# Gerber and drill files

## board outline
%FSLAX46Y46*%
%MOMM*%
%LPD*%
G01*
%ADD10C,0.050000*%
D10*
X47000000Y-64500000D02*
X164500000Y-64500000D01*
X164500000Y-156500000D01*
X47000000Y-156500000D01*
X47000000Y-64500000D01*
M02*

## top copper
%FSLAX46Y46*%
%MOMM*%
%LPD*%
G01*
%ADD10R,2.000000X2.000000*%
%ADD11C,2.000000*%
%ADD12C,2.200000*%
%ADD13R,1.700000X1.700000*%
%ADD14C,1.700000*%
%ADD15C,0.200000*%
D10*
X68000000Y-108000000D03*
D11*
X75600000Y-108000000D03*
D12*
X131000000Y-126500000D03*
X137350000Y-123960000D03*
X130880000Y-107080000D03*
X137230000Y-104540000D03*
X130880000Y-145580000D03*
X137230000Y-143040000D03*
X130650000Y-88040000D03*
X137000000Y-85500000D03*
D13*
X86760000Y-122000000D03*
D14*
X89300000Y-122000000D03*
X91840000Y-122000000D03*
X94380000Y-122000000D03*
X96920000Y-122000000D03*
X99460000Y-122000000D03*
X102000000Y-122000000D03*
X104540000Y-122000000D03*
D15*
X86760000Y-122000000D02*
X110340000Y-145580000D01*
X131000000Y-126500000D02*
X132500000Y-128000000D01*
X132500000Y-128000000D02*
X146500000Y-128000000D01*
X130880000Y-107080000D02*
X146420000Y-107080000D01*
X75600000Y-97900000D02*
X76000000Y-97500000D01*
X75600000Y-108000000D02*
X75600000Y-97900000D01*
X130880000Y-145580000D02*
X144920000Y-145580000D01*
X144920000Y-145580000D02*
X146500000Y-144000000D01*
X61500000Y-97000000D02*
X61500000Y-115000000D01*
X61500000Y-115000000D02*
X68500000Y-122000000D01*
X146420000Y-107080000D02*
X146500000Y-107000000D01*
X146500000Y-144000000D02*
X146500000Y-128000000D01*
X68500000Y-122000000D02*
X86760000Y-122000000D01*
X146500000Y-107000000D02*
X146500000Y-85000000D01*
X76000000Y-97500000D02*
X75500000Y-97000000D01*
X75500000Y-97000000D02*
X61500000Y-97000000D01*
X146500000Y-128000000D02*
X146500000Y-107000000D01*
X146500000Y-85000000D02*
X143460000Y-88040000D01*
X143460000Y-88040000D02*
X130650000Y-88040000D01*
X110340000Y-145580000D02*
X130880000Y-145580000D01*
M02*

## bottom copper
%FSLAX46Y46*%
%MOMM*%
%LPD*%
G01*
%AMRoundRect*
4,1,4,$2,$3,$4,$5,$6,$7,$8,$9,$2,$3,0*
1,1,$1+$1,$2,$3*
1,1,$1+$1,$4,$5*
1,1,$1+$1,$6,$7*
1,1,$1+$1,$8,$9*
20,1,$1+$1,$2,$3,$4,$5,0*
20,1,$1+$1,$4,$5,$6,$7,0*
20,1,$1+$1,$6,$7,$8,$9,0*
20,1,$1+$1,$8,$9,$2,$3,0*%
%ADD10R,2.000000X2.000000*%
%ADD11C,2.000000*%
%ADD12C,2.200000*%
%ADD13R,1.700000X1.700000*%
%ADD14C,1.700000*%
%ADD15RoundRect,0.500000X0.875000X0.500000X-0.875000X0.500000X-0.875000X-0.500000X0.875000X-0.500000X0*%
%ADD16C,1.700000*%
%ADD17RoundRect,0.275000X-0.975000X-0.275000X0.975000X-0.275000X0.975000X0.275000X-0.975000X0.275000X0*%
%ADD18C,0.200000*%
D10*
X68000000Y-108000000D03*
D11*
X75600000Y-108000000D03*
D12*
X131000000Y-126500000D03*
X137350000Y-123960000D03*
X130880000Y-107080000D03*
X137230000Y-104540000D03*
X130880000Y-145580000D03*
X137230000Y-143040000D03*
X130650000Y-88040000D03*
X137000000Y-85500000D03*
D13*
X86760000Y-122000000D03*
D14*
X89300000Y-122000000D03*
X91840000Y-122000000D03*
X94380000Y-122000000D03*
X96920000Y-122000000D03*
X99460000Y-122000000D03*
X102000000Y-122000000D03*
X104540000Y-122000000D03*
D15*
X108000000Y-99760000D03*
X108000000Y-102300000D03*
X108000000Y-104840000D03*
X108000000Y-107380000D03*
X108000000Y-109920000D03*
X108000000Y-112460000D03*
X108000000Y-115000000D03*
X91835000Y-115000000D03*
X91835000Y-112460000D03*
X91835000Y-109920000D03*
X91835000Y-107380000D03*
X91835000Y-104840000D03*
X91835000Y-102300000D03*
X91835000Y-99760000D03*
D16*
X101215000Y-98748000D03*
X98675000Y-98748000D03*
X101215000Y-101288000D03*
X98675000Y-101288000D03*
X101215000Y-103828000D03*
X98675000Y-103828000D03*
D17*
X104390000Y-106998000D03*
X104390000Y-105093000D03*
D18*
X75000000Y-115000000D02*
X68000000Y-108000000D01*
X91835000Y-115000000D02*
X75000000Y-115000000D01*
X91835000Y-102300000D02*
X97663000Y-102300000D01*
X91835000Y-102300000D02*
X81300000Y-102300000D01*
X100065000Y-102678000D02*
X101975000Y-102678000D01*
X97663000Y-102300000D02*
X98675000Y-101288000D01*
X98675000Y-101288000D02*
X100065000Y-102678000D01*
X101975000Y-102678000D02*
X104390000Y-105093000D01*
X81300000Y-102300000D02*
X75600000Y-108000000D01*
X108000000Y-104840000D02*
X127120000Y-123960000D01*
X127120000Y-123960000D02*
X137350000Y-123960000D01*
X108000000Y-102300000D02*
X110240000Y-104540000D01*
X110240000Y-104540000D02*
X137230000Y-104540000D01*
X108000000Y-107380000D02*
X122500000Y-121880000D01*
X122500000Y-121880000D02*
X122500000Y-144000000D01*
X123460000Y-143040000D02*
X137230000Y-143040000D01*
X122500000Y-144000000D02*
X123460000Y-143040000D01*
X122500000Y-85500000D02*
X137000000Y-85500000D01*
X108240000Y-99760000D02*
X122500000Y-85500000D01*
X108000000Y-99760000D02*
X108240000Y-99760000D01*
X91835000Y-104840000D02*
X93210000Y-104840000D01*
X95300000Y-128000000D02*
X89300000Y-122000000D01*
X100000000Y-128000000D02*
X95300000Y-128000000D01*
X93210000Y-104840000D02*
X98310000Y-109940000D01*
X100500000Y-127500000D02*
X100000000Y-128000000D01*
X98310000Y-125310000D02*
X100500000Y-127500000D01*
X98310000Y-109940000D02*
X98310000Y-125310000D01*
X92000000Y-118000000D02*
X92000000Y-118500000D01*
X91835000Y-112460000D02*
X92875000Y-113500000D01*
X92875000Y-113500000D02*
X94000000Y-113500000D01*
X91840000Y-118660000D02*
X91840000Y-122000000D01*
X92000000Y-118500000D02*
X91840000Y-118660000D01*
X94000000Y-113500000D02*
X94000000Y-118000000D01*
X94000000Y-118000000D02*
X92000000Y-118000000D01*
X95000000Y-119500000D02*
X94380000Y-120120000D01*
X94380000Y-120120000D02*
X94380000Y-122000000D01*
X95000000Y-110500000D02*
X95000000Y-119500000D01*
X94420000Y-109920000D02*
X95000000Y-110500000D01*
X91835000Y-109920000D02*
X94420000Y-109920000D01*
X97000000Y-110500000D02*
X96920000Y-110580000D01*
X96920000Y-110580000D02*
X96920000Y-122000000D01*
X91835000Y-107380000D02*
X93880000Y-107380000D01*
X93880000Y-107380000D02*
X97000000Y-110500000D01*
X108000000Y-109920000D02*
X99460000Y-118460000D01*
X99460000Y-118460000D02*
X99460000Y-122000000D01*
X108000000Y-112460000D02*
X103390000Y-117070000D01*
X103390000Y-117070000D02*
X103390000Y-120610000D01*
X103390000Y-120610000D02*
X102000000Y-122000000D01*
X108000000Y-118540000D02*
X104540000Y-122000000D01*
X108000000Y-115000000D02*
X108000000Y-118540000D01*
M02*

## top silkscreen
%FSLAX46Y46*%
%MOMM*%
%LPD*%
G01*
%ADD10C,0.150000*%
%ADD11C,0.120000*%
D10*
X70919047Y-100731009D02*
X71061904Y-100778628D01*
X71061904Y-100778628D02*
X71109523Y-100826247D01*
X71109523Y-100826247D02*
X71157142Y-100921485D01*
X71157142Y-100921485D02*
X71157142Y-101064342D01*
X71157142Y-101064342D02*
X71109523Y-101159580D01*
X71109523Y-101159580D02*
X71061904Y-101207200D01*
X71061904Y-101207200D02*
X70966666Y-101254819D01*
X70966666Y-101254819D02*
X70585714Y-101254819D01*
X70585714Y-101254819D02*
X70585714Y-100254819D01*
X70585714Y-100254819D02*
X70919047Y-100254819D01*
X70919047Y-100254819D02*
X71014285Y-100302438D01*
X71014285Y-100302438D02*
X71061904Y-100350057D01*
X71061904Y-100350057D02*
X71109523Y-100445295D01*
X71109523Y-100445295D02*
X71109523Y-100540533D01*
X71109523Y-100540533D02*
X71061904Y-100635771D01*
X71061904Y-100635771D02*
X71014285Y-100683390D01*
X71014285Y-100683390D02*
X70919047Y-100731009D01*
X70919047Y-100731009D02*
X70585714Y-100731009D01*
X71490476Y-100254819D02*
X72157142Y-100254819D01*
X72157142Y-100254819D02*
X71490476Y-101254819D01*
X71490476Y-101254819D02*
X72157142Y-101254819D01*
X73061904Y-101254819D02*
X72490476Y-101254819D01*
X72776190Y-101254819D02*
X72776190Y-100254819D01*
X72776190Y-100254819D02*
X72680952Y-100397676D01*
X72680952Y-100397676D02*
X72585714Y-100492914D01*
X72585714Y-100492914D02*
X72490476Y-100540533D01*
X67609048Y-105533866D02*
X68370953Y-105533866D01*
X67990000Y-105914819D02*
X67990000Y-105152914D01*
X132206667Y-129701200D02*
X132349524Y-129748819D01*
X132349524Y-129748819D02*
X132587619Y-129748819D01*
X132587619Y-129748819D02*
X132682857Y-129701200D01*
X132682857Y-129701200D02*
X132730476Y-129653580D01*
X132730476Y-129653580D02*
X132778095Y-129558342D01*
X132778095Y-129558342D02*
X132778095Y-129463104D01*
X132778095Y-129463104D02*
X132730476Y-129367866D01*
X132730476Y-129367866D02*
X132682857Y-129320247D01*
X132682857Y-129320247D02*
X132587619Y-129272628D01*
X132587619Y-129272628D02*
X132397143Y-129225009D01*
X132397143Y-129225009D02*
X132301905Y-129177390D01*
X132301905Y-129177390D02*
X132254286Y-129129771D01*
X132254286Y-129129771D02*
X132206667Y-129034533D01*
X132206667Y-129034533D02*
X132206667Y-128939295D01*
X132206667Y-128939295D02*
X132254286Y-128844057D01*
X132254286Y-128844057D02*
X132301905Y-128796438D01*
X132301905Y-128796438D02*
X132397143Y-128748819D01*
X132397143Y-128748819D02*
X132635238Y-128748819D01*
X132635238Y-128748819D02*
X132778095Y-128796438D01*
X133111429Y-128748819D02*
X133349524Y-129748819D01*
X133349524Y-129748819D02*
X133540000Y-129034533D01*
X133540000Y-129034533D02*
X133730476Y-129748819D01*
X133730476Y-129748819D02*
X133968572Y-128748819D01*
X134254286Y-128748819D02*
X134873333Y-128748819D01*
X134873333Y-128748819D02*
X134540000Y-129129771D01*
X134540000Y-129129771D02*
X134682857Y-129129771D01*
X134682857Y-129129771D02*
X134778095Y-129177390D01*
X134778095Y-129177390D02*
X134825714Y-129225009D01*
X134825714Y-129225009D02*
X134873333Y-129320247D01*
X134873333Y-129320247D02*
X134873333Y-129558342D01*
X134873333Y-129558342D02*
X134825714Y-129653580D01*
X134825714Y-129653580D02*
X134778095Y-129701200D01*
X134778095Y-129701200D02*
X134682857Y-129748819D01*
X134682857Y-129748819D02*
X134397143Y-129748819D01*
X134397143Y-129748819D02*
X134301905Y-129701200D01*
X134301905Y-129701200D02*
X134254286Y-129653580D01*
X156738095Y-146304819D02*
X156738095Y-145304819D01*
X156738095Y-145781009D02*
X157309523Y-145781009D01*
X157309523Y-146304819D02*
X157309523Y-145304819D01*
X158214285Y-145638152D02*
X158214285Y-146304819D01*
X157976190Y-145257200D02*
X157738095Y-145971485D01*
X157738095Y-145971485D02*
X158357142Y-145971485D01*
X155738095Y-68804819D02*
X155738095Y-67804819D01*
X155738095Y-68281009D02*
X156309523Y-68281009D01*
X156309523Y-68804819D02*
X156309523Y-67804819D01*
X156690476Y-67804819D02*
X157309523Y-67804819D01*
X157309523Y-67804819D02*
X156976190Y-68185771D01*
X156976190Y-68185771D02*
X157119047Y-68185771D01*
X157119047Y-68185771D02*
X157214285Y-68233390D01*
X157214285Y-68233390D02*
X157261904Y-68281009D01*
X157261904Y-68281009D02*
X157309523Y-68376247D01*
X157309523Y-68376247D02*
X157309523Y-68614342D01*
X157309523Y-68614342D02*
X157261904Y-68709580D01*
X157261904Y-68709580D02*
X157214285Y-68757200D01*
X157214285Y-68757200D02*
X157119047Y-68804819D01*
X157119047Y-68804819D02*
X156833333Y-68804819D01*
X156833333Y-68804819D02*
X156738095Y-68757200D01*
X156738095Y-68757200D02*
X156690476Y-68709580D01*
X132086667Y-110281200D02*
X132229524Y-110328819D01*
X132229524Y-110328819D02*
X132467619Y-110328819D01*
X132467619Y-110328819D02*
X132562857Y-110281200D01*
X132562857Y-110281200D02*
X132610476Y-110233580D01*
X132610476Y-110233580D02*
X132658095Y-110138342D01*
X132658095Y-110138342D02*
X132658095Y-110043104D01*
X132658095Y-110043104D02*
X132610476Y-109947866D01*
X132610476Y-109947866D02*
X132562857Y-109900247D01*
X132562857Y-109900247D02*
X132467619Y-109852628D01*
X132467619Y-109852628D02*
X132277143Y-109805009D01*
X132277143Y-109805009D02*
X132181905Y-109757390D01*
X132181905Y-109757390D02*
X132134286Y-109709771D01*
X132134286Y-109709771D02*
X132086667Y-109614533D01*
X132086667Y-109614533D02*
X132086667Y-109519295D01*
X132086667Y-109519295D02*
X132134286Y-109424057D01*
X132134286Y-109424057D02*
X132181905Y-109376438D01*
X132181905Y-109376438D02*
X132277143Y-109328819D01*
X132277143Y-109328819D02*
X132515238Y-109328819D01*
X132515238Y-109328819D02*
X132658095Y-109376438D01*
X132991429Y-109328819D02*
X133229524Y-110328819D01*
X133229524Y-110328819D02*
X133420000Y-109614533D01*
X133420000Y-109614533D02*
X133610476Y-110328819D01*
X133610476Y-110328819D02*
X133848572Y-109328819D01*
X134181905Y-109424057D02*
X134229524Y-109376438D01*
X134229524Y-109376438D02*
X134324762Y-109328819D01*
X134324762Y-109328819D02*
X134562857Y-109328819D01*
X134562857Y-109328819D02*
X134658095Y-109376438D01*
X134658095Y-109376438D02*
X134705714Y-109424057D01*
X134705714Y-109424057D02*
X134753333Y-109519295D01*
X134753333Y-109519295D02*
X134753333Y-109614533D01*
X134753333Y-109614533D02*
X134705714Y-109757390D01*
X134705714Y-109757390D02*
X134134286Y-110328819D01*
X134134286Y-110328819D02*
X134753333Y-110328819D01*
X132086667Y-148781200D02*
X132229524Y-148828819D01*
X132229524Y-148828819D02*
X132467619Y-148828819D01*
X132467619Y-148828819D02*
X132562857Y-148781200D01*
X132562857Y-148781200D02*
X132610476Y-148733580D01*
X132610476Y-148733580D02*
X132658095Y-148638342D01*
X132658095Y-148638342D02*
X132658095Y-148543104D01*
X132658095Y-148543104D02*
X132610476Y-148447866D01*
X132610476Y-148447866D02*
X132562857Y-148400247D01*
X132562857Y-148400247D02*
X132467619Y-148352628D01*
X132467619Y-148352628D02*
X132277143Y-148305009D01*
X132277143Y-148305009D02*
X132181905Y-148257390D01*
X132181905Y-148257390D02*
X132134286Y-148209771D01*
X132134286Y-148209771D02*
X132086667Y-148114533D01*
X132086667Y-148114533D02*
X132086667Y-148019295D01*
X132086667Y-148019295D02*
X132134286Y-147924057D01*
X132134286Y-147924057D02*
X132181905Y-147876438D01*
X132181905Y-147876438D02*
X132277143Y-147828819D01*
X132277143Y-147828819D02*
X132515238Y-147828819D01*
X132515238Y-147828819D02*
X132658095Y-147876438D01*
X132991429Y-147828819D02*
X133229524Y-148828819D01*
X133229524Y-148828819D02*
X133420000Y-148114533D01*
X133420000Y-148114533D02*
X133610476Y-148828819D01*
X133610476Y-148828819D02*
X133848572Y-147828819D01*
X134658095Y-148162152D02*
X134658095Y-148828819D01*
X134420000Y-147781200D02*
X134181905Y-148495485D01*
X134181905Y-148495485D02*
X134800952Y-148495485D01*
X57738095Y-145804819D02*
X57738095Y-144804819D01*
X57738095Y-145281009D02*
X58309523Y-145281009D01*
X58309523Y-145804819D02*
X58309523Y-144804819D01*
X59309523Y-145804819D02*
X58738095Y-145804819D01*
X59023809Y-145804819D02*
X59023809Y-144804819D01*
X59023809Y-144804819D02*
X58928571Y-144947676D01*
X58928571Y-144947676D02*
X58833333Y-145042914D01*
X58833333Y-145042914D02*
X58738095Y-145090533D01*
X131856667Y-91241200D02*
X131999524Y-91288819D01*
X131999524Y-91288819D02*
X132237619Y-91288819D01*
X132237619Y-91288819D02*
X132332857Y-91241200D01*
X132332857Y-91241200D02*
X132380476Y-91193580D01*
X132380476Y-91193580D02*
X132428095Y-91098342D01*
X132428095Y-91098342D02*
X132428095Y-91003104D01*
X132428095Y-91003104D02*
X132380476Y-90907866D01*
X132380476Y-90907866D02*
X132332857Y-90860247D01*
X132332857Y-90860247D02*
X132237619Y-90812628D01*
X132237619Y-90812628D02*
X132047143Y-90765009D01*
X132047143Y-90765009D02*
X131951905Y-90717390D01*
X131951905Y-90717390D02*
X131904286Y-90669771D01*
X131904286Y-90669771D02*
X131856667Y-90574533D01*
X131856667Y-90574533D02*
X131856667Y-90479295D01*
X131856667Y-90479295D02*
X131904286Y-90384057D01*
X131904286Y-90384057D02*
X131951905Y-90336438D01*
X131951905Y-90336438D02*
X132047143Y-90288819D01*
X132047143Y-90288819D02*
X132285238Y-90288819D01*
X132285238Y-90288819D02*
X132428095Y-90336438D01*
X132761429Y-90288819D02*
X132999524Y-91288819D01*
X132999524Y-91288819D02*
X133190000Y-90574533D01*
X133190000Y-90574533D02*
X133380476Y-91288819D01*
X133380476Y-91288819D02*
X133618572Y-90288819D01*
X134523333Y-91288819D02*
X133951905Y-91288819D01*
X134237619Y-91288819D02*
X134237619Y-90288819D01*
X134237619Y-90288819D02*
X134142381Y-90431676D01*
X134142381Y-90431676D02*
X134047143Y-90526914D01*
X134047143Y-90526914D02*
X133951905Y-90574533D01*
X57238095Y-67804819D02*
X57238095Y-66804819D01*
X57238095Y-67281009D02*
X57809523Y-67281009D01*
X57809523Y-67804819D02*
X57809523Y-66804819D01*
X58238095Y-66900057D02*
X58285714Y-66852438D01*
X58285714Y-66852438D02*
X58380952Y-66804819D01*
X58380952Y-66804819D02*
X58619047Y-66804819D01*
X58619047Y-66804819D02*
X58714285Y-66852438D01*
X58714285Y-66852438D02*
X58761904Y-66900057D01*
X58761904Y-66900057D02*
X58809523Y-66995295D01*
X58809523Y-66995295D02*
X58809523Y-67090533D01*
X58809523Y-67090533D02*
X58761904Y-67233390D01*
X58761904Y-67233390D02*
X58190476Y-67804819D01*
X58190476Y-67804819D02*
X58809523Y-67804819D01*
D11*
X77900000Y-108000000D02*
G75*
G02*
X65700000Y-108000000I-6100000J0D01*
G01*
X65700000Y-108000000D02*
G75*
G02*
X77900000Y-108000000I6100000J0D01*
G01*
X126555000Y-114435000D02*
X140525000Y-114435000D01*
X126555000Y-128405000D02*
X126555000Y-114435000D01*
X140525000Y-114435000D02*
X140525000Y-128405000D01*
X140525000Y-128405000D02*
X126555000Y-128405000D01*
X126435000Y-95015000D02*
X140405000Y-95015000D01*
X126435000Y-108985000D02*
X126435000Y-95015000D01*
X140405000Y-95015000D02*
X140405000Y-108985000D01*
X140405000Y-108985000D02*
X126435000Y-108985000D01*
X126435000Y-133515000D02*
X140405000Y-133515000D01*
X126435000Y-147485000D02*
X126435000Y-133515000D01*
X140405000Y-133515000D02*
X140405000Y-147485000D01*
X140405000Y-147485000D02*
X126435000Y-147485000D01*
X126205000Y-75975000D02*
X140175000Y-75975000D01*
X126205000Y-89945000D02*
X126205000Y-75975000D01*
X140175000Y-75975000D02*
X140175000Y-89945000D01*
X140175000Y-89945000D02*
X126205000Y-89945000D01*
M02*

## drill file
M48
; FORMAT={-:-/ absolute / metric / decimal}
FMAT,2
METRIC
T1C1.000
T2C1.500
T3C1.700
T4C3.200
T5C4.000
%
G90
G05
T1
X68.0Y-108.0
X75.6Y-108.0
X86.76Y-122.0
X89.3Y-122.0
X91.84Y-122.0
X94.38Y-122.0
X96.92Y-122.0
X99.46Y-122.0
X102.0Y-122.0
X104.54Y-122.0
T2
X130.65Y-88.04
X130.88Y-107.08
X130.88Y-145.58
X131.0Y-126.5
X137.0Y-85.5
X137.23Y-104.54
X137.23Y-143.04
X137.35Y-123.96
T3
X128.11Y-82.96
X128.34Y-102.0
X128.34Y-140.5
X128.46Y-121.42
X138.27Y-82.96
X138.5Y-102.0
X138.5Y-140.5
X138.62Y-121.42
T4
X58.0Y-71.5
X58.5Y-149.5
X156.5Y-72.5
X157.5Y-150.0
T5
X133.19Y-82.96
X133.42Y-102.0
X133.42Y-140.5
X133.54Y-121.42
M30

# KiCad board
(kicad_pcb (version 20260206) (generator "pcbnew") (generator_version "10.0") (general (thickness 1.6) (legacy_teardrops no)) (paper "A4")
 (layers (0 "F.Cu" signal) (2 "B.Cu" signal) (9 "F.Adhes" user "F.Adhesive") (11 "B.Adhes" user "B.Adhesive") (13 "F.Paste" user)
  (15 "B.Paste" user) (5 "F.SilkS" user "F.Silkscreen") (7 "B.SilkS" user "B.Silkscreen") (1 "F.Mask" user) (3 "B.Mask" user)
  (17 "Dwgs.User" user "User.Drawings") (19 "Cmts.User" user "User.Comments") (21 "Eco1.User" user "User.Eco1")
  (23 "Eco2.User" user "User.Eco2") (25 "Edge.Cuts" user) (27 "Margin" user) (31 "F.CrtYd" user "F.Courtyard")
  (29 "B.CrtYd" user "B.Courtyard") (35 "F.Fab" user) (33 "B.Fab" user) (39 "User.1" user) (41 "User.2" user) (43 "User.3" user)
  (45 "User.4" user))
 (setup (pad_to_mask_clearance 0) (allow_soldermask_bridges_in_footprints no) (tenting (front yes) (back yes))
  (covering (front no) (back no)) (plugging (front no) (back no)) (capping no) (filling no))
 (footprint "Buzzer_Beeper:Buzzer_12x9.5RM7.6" (layer "F.Cu") (at 68 108)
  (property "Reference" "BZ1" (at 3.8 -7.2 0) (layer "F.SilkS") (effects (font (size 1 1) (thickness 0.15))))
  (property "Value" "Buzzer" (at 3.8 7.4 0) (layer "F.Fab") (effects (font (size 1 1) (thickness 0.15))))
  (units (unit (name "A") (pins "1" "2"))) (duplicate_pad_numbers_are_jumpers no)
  (fp_circle (center 3.8 0) (end 9.9 0) (stroke (width 0.12) (type solid)) (fill no) (layer "F.SilkS"))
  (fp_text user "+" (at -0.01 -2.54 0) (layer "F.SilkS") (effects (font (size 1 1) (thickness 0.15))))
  (pad "1" thru_hole rect (at 0 0) (size 2 2) (drill 1) (layers "*.Cu" "*.Mask") (remove_unused_layers no) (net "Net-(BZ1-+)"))
  (pad "2" thru_hole circle (at 7.6 0) (size 2 2) (drill 1) (layers "*.Cu" "*.Mask") (remove_unused_layers no) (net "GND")))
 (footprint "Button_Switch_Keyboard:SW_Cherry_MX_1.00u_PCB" (layer "F.Cu") (at 131 126.5 180)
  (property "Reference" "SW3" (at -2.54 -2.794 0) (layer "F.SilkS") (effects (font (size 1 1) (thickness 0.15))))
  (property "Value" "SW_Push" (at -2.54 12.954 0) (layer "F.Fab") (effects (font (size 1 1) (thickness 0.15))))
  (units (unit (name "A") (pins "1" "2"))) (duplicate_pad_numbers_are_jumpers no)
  (fp_line (start 4.445 12.065) (end -9.525 12.065) (stroke (width 0.12) (type solid)) (layer "F.SilkS"))
  (fp_line (start 4.445 -1.905) (end 4.445 12.065) (stroke (width 0.12) (type solid)) (layer "F.SilkS"))
  (fp_line (start -9.525 12.065) (end -9.525 -1.905) (stroke (width 0.12) (type solid)) (layer "F.SilkS"))
  (fp_line (start -9.525 -1.905) (end 4.445 -1.905) (stroke (width 0.12) (type solid)) (layer "F.SilkS"))
  (pad "" np_thru_hole circle (at -7.62 5.08 180) (size 1.7 1.7) (drill 1.7) (layers "*.Cu" "*.Mask"))
  (pad "" np_thru_hole circle (at -2.54 5.08 180) (size 4 4) (drill 4) (layers "*.Cu" "*.Mask"))
  (pad "" np_thru_hole circle (at 2.54 5.08 180) (size 1.7 1.7) (drill 1.7) (layers "*.Cu" "*.Mask"))
  (pad "1" thru_hole circle (at 0 0 180) (size 2.2 2.2) (drill 1.5) (layers "*.Cu" "*.Mask") (remove_unused_layers no) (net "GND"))
  (pad "2" thru_hole circle (at -6.35 2.54 180) (size 2.2 2.2) (drill 1.5) (layers "*.Cu" "*.Mask") (remove_unused_layers no)
   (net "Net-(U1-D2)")))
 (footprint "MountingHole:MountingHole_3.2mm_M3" (layer "F.Cu") (at 157.5 150)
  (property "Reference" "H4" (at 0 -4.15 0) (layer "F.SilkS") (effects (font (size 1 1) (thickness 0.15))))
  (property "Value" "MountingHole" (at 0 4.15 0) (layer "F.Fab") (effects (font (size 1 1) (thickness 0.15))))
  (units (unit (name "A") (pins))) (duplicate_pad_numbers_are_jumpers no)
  (pad "" np_thru_hole circle (at 0 0) (size 3.2 3.2) (drill 3.2) (layers "*.Cu" "*.Mask")))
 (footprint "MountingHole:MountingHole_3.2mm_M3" (layer "F.Cu") (at 156.5 72.5)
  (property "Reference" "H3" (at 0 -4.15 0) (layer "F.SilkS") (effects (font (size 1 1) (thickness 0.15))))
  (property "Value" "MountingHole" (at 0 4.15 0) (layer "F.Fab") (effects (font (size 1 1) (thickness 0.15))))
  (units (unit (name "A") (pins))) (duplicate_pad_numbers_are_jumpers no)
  (pad "" np_thru_hole circle (at 0 0) (size 3.2 3.2) (drill 3.2) (layers "*.Cu" "*.Mask")))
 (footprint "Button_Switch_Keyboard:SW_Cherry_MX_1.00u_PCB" (layer "F.Cu") (at 130.88 107.08 180)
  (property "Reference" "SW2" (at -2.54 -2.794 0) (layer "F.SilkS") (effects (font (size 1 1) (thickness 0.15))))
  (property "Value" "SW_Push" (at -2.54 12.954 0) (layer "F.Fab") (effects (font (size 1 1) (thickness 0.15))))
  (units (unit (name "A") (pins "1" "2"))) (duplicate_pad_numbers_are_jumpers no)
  (fp_line (start 4.445 12.065) (end -9.525 12.065) (stroke (width 0.12) (type solid)) (layer "F.SilkS"))
  (fp_line (start 4.445 -1.905) (end 4.445 12.065) (stroke (width 0.12) (type solid)) (layer "F.SilkS"))
  (fp_line (start -9.525 12.065) (end -9.525 -1.905) (stroke (width 0.12) (type solid)) (layer "F.SilkS"))
  (fp_line (start -9.525 -1.905) (end 4.445 -1.905) (stroke (width 0.12) (type solid)) (layer "F.SilkS"))
  (pad "" np_thru_hole circle (at -7.62 5.08 180) (size 1.7 1.7) (drill 1.7) (layers "*.Cu" "*.Mask"))
  (pad "" np_thru_hole circle (at -2.54 5.08 180) (size 4 4) (drill 4) (layers "*.Cu" "*.Mask"))
  (pad "" np_thru_hole circle (at 2.54 5.08 180) (size 1.7 1.7) (drill 1.7) (layers "*.Cu" "*.Mask"))
  (pad "1" thru_hole circle (at 0 0 180) (size 2.2 2.2) (drill 1.5) (layers "*.Cu" "*.Mask") (remove_unused_layers no) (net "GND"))
  (pad "2" thru_hole circle (at -6.35 2.54 180) (size 2.2 2.2) (drill 1.5) (layers "*.Cu" "*.Mask") (remove_unused_layers no)
   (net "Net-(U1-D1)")))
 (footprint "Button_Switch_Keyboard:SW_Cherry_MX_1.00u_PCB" (layer "F.Cu") (at 130.88 145.58 180)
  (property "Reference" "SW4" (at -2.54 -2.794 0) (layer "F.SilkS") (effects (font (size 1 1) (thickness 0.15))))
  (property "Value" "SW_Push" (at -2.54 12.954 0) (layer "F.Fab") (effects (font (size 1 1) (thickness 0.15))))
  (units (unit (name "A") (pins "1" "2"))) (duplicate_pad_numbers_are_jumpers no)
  (fp_line (start 4.445 12.065) (end -9.525 12.065) (stroke (width 0.12) (type solid)) (layer "F.SilkS"))
  (fp_line (start 4.445 -1.905) (end 4.445 12.065) (stroke (width 0.12) (type solid)) (layer "F.SilkS"))
  (fp_line (start -9.525 12.065) (end -9.525 -1.905) (stroke (width 0.12) (type solid)) (layer "F.SilkS"))
  (fp_line (start -9.525 -1.905) (end 4.445 -1.905) (stroke (width 0.12) (type solid)) (layer "F.SilkS"))
  (pad "" np_thru_hole circle (at -7.62 5.08 180) (size 1.7 1.7) (drill 1.7) (layers "*.Cu" "*.Mask"))
  (pad "" np_thru_hole circle (at -2.54 5.08 180) (size 4 4) (drill 4) (layers "*.Cu" "*.Mask"))
  (pad "" np_thru_hole circle (at 2.54 5.08 180) (size 1.7 1.7) (drill 1.7) (layers "*.Cu" "*.Mask"))
  (pad "1" thru_hole circle (at 0 0 180) (size 2.2 2.2) (drill 1.5) (layers "*.Cu" "*.Mask") (remove_unused_layers no) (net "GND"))
  (pad "2" thru_hole circle (at -6.35 2.54 180) (size 2.2 2.2) (drill 1.5) (layers "*.Cu" "*.Mask") (remove_unused_layers no)
   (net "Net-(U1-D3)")))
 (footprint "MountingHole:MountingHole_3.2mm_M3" (layer "F.Cu") (at 58.5 149.5)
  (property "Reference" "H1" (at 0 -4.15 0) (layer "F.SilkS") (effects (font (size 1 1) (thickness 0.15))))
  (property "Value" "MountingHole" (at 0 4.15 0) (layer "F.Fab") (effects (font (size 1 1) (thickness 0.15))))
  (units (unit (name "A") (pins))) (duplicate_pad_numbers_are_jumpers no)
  (pad "" np_thru_hole circle (at 0 0) (size 3.2 3.2) (drill 3.2) (layers "*.Cu" "*.Mask")))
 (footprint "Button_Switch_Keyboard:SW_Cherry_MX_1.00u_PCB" (layer "F.Cu") (at 130.65 88.04 180)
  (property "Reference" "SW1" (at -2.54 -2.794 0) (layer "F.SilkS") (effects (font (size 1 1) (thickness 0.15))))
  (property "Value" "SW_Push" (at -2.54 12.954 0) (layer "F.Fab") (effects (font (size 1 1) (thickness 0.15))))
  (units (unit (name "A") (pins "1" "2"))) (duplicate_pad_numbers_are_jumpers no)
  (fp_line (start 4.445 12.065) (end -9.525 12.065) (stroke (width 0.12) (type solid)) (layer "F.SilkS"))
  (fp_line (start 4.445 -1.905) (end 4.445 12.065) (stroke (width 0.12) (type solid)) (layer "F.SilkS"))
  (fp_line (start -9.525 12.065) (end -9.525 -1.905) (stroke (width 0.12) (type solid)) (layer "F.SilkS"))
  (fp_line (start -9.525 -1.905) (end 4.445 -1.905) (stroke (width 0.12) (type solid)) (layer "F.SilkS"))
  (pad "" np_thru_hole circle (at -7.62 5.08 180) (size 1.7 1.7) (drill 1.7) (layers "*.Cu" "*.Mask"))
  (pad "" np_thru_hole circle (at -2.54 5.08 180) (size 4 4) (drill 4) (layers "*.Cu" "*.Mask"))
  (pad "" np_thru_hole circle (at 2.54 5.08 180) (size 1.7 1.7) (drill 1.7) (layers "*.Cu" "*.Mask"))
  (pad "1" thru_hole circle (at 0 0 180) (size 2.2 2.2) (drill 1.5) (layers "*.Cu" "*.Mask") (remove_unused_layers no) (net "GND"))
  (pad "2" thru_hole circle (at -6.35 2.54 180) (size 2.2 2.2) (drill 1.5) (layers "*.Cu" "*.Mask") (remove_unused_layers no)
   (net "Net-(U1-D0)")))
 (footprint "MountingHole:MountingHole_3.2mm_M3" (layer "F.Cu") (at 58 71.5)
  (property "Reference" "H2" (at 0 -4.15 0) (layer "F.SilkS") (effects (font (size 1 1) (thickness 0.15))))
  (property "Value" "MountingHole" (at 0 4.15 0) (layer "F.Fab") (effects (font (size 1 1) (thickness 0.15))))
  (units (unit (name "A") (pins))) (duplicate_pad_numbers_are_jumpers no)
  (pad "" np_thru_hole circle (at 0 0) (size 3.2 3.2) (drill 3.2) (layers "*.Cu" "*.Mask")))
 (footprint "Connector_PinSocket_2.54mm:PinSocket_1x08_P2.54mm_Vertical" (layer "B.Cu") (at 86.76 122 -90)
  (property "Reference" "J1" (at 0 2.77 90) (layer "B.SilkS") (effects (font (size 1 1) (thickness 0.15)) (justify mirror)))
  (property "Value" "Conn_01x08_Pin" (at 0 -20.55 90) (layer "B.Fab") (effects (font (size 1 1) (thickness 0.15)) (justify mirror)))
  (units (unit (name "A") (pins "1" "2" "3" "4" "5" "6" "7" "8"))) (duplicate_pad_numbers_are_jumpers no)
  (pad "1" thru_hole rect (at 0 0 270) (size 1.7 1.7) (drill 1) (layers "*.Cu" "*.Mask") (remove_unused_layers no) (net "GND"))
  (pad "2" thru_hole circle (at 0 -2.54 270) (size 1.7 1.7) (drill 1) (layers "*.Cu" "*.Mask") (remove_unused_layers no) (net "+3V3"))
  (pad "3" thru_hole circle (at 0 -5.08 270) (size 1.7 1.7) (drill 1) (layers "*.Cu" "*.Mask") (remove_unused_layers no) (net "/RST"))
  (pad "4" thru_hole circle (at 0 -7.62 270) (size 1.7 1.7) (drill 1) (layers "*.Cu" "*.Mask") (remove_unused_layers no) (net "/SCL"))
  (pad "5" thru_hole circle (at 0 -10.16 270) (size 1.7 1.7) (drill 1) (layers "*.Cu" "*.Mask") (remove_unused_layers no) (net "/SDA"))
  (pad "6" thru_hole circle (at 0 -12.7 270) (size 1.7 1.7) (drill 1) (layers "*.Cu" "*.Mask") (remove_unused_layers no) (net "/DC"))
  (pad "7" thru_hole circle (at 0 -15.24 270) (size 1.7 1.7) (drill 1) (layers "*.Cu" "*.Mask") (remove_unused_layers no) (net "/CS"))
  (pad "8" thru_hole circle (at 0 -17.78 270) (size 1.7 1.7) (drill 1) (layers "*.Cu" "*.Mask") (remove_unused_layers no) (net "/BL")))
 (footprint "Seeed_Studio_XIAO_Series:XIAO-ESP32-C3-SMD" (layer "B.Cu") (at 108.835 117.88 180)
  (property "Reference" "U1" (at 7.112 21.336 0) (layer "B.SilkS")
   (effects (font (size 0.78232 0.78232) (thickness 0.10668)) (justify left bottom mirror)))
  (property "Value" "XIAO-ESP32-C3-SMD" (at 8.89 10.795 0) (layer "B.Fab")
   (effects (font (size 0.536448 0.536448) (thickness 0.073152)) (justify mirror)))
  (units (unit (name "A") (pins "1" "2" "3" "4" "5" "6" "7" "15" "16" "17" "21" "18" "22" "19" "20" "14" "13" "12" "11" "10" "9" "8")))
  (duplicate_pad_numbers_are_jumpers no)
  (pad "1" smd roundrect (at 0.835 18.12 180) (size 2.75 2) (layers "B.Cu" "B.Mask" "B.Paste") (roundrect_rratio 0.25) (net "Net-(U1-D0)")
   (solder_mask_margin 0.0508) (thermal_bridge_angle 45))
  (pad "2" smd roundrect (at 0.835 15.58 180) (size 2.75 2) (layers "B.Cu" "B.Mask" "B.Paste") (roundrect_rratio 0.25) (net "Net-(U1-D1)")
   (solder_mask_margin 0.0508) (thermal_bridge_angle 45))
  (pad "3" smd roundrect (at 0.835 13.04 180) (size 2.75 2) (layers "B.Cu" "B.Mask" "B.Paste") (roundrect_rratio 0.25) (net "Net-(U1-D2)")
   (solder_mask_margin 0.0508) (thermal_bridge_angle 45))
  (pad "4" smd roundrect (at 0.835 10.5 180) (size 2.75 2) (layers "B.Cu" "B.Mask" "B.Paste") (roundrect_rratio 0.25) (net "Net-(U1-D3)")
   (solder_mask_margin 0.0508) (thermal_bridge_angle 45))
  (pad "5" smd roundrect (at 0.835 7.96 180) (size 2.75 2) (layers "B.Cu" "B.Mask" "B.Paste") (roundrect_rratio 0.25) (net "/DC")
   (solder_mask_margin 0.0508) (thermal_bridge_angle 45))
  (pad "6" smd roundrect (at 0.835 5.42 180) (size 2.75 2) (layers "B.Cu" "B.Mask" "B.Paste") (roundrect_rratio 0.25) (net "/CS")
   (solder_mask_margin 0.0508) (thermal_bridge_angle 45))
  (pad "7" smd roundrect (at 0.835 2.88 180) (size 2.75 2) (layers "B.Cu" "B.Mask" "B.Paste") (roundrect_rratio 0.25) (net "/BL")
   (solder_mask_margin 0.0508) (thermal_bridge_angle 45))
  (pad "8" smd roundrect (at 17 2.88 180) (size 2.75 2) (layers "B.Cu" "B.Mask" "B.Paste") (roundrect_rratio 0.25) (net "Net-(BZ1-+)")
   (solder_mask_margin 0.0508) (thermal_bridge_angle 45))
  (pad "9" smd roundrect (at 17 5.42 180) (size 2.75 2) (layers "B.Cu" "B.Mask" "B.Paste") (roundrect_rratio 0.25) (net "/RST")
   (solder_mask_margin 0.0508) (thermal_bridge_angle 45))
  (pad "10" smd roundrect (at 17 7.96 180) (size 2.75 2) (layers "B.Cu" "B.Mask" "B.Paste") (roundrect_rratio 0.25) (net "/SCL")
   (solder_mask_margin 0.0508) (thermal_bridge_angle 45))
  (pad "11" smd roundrect (at 17 10.5 180) (size 2.75 2) (layers "B.Cu" "B.Mask" "B.Paste") (roundrect_rratio 0.25) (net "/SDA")
   (solder_mask_margin 0.0508) (thermal_bridge_angle 45))
  (pad "12" smd roundrect (at 17 13.04 180) (size 2.75 2) (layers "B.Cu" "B.Mask" "B.Paste") (roundrect_rratio 0.25) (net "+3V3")
   (solder_mask_margin 0.0508) (thermal_bridge_angle 45))
  (pad "13" smd roundrect (at 17 15.58 180) (size 2.75 2) (layers "B.Cu" "B.Mask" "B.Paste") (roundrect_rratio 0.25) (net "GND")
   (solder_mask_margin 0.0508) (thermal_bridge_angle 45))
  (pad "14" smd roundrect (at 17 18.12 180) (size 2.75 2) (layers "B.Cu" "B.Mask" "B.Paste") (roundrect_rratio 0.25)
   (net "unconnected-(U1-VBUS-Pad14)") (solder_mask_margin 0.0508) (thermal_bridge_angle 45))
  (pad "15" smd circle (at 7.62 19.132 180) (size 1.7 1.7) (layers "B.Cu" "B.Mask" "B.Paste") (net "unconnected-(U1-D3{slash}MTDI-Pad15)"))
  (pad "16" smd circle (at 10.16 19.132 180) (size 1.7 1.7) (layers "B.Cu" "B.Mask" "B.Paste") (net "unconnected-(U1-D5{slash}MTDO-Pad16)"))
  (pad "17" smd circle (at 7.62 16.592 180) (size 1.7 1.7) (layers "B.Cu" "B.Mask" "B.Paste") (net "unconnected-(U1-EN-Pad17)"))
  (pad "18" smd circle (at 10.16 16.592 180) (size 1.7 1.7) (layers "B.Cu" "B.Mask" "B.Paste") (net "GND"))
  (pad "19" smd circle (at 7.62 14.052 180) (size 1.7 1.7) (layers "B.Cu" "B.Mask" "B.Paste") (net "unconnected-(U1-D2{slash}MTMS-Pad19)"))
  (pad "20" smd circle (at 10.16 14.052 180) (size 1.7 1.7) (layers "B.Cu" "B.Mask" "B.Paste") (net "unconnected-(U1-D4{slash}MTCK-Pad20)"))
  (pad "21" smd roundrect (at 4.445 10.882) (size 2.5 1.1) (layers "B.Cu" "B.Mask" "B.Paste") (roundrect_rratio 0.25)
   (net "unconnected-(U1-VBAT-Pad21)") (thermal_bridge_angle 45))
  (pad "22" smd roundrect (at 4.445 12.787) (size 2.5 1.1) (layers "B.Cu" "B.Mask" "B.Paste") (roundrect_rratio 0.25) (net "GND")
   (thermal_bridge_angle 45)))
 (gr_rect (start 47 64.5) (end 164.5 156.5) (stroke (width 0.05) (type default)) (fill no) (layer "Edge.Cuts"))
 (segment (start 75 115) (end 68 108) (width 0.2) (layer "B.Cu") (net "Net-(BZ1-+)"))
 (segment (start 91.835 115) (end 75 115) (width 0.2) (layer "B.Cu") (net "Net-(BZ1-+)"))
 (segment (start 86.76 122) (end 110.34 145.58) (width 0.2) (layer "F.Cu") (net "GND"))
 (segment (start 131 126.5) (end 132.5 128) (width 0.2) (layer "F.Cu") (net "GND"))
 (segment (start 132.5 128) (end 146.5 128) (width 0.2) (layer "F.Cu") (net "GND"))
 (segment (start 130.88 107.08) (end 146.42 107.08) (width 0.2) (layer "F.Cu") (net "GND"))
 (segment (start 75.6 97.9) (end 76 97.5) (width 0.2) (layer "F.Cu") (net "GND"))
 (segment (start 75.6 108) (end 75.6 97.9) (width 0.2) (layer "F.Cu") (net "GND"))
 (segment (start 130.88 145.58) (end 144.92 145.58) (width 0.2) (layer "F.Cu") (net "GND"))
 (segment (start 144.92 145.58) (end 146.5 144) (width 0.2) (layer "F.Cu") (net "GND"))
 (segment (start 61.5 97) (end 61.5 115) (width 0.2) (layer "F.Cu") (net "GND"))
 (segment (start 61.5 115) (end 68.5 122) (width 0.2) (layer "F.Cu") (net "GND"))
 (segment (start 146.42 107.08) (end 146.5 107) (width 0.2) (layer "F.Cu") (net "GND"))
 (segment (start 146.5 144) (end 146.5 128) (width 0.2) (layer "F.Cu") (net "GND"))
 (segment (start 68.5 122) (end 86.76 122) (width 0.2) (layer "F.Cu") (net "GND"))
 (segment (start 146.5 107) (end 146.5 85) (width 0.2) (layer "F.Cu") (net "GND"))
 (segment (start 76 97.5) (end 75.5 97) (width 0.2) (layer "F.Cu") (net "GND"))
 (segment (start 75.5 97) (end 61.5 97) (width 0.2) (layer "F.Cu") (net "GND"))
 (segment (start 146.5 128) (end 146.5 107) (width 0.2) (layer "F.Cu") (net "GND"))
 (segment (start 146.5 85) (end 143.46 88.04) (width 0.2) (layer "F.Cu") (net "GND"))
 (segment (start 143.46 88.04) (end 130.65 88.04) (width 0.2) (layer "F.Cu") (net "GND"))
 (segment (start 110.34 145.58) (end 130.88 145.58) (width 0.2) (layer "F.Cu") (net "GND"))
 (segment (start 91.835 102.3) (end 97.663 102.3) (width 0.2) (layer "B.Cu") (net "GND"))
 (segment (start 91.835 102.3) (end 81.3 102.3) (width 0.2) (layer "B.Cu") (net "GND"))
 (segment (start 100.065 102.678) (end 101.975 102.678) (width 0.2) (layer "B.Cu") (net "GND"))
 (segment (start 97.663 102.3) (end 98.675 101.288) (width 0.2) (layer "B.Cu") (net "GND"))
 (segment (start 98.675 101.288) (end 100.065 102.678) (width 0.2) (layer "B.Cu") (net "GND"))
 (segment (start 101.975 102.678) (end 104.39 105.093) (width 0.2) (layer "B.Cu") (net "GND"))
 (segment (start 81.3 102.3) (end 75.6 108) (width 0.2) (layer "B.Cu") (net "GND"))
 (segment (start 108 104.84) (end 127.12 123.96) (width 0.2) (layer "B.Cu") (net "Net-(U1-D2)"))
 (segment (start 127.12 123.96) (end 137.35 123.96) (width 0.2) (layer "B.Cu") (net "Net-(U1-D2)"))
 (segment (start 108 102.3) (end 110.24 104.54) (width 0.2) (layer "B.Cu") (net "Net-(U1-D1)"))
 (segment (start 110.24 104.54) (end 137.23 104.54) (width 0.2) (layer "B.Cu") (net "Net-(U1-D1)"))
 (segment (start 108 107.38) (end 122.5 121.88) (width 0.2) (layer "B.Cu") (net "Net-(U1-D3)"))
 (segment (start 122.5 121.88) (end 122.5 144) (width 0.2) (layer "B.Cu") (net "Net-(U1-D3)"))
 (segment (start 123.46 143.04) (end 137.23 143.04) (width 0.2) (layer "B.Cu") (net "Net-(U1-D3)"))
 (segment (start 122.5 144) (end 123.46 143.04) (width 0.2) (layer "B.Cu") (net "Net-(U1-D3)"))
 (segment (start 122.5 85.5) (end 137 85.5) (width 0.2) (layer "B.Cu") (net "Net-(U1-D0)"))
 (segment (start 108.24 99.76) (end 122.5 85.5) (width 0.2) (layer "B.Cu") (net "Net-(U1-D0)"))
 (segment (start 108 99.76) (end 108.24 99.76) (width 0.2) (layer "B.Cu") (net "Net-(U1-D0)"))
 (segment (start 91.835 104.84) (end 93.21 104.84) (width 0.2) (layer "B.Cu") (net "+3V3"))
 (segment (start 95.3 128) (end 89.3 122) (width 0.2) (layer "B.Cu") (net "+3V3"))
 (segment (start 100 128) (end 95.3 128) (width 0.2) (layer "B.Cu") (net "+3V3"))
 (segment (start 93.21 104.84) (end 98.31 109.94) (width 0.2) (layer "B.Cu") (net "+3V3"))
 (segment (start 100.5 127.5) (end 100 128) (width 0.2) (layer "B.Cu") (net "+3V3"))
 (segment (start 98.31 125.31) (end 100.5 127.5) (width 0.2) (layer "B.Cu") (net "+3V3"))
 (segment (start 98.31 109.94) (end 98.31 125.31) (width 0.2) (layer "B.Cu") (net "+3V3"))
 (segment (start 92 118) (end 92 118.5) (width 0.2) (layer "B.Cu") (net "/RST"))
 (segment (start 91.835 112.46) (end 92.875 113.5) (width 0.2) (layer "B.Cu") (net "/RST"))
 (segment (start 92.875 113.5) (end 94 113.5) (width 0.2) (layer "B.Cu") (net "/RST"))
 (segment (start 91.84 118.66) (end 91.84 122) (width 0.2) (layer "B.Cu") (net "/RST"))
 (segment (start 92 118.5) (end 91.84 118.66) (width 0.2) (layer "B.Cu") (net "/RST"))
 (segment (start 94 113.5) (end 94 118) (width 0.2) (layer "B.Cu") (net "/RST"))
 (segment (start 94 118) (end 92 118) (width 0.2) (layer "B.Cu") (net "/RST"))
 (segment (start 95 119.5) (end 94.38 120.12) (width 0.2) (layer "B.Cu") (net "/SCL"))
 (segment (start 94.38 120.12) (end 94.38 122) (width 0.2) (layer "B.Cu") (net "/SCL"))
 (segment (start 95 110.5) (end 95 119.5) (width 0.2) (layer "B.Cu") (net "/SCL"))
 (segment (start 94.42 109.92) (end 95 110.5) (width 0.2) (layer "B.Cu") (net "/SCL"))
 (segment (start 91.835 109.92) (end 94.42 109.92) (width 0.2) (layer "B.Cu") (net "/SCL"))
 (segment (start 97 110.5) (end 96.92 110.58) (width 0.2) (layer "B.Cu") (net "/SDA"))
 (segment (start 96.92 110.58) (end 96.92 122) (width 0.2) (layer "B.Cu") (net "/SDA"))
 (segment (start 91.835 107.38) (end 93.88 107.38) (width 0.2) (layer "B.Cu") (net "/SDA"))
 (segment (start 93.88 107.38) (end 97 110.5) (width 0.2) (layer "B.Cu") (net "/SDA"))
 (segment (start 108 109.92) (end 99.46 118.46) (width 0.2) (layer "B.Cu") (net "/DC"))
 (segment (start 99.46 118.46) (end 99.46 122) (width 0.2) (layer "B.Cu") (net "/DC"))
 (segment (start 108 112.46) (end 103.39 117.07) (width 0.2) (layer "B.Cu") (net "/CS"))
 (segment (start 103.39 117.07) (end 103.39 120.61) (width 0.2) (layer "B.Cu") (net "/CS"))
 (segment (start 103.39 120.61) (end 102 122) (width 0.2) (layer "B.Cu") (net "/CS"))
 (segment (start 108 118.54) (end 104.54 122) (width 0.2) (layer "B.Cu") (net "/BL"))
 (segment (start 108 115) (end 108 118.54) (width 0.2) (layer "B.Cu") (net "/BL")))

